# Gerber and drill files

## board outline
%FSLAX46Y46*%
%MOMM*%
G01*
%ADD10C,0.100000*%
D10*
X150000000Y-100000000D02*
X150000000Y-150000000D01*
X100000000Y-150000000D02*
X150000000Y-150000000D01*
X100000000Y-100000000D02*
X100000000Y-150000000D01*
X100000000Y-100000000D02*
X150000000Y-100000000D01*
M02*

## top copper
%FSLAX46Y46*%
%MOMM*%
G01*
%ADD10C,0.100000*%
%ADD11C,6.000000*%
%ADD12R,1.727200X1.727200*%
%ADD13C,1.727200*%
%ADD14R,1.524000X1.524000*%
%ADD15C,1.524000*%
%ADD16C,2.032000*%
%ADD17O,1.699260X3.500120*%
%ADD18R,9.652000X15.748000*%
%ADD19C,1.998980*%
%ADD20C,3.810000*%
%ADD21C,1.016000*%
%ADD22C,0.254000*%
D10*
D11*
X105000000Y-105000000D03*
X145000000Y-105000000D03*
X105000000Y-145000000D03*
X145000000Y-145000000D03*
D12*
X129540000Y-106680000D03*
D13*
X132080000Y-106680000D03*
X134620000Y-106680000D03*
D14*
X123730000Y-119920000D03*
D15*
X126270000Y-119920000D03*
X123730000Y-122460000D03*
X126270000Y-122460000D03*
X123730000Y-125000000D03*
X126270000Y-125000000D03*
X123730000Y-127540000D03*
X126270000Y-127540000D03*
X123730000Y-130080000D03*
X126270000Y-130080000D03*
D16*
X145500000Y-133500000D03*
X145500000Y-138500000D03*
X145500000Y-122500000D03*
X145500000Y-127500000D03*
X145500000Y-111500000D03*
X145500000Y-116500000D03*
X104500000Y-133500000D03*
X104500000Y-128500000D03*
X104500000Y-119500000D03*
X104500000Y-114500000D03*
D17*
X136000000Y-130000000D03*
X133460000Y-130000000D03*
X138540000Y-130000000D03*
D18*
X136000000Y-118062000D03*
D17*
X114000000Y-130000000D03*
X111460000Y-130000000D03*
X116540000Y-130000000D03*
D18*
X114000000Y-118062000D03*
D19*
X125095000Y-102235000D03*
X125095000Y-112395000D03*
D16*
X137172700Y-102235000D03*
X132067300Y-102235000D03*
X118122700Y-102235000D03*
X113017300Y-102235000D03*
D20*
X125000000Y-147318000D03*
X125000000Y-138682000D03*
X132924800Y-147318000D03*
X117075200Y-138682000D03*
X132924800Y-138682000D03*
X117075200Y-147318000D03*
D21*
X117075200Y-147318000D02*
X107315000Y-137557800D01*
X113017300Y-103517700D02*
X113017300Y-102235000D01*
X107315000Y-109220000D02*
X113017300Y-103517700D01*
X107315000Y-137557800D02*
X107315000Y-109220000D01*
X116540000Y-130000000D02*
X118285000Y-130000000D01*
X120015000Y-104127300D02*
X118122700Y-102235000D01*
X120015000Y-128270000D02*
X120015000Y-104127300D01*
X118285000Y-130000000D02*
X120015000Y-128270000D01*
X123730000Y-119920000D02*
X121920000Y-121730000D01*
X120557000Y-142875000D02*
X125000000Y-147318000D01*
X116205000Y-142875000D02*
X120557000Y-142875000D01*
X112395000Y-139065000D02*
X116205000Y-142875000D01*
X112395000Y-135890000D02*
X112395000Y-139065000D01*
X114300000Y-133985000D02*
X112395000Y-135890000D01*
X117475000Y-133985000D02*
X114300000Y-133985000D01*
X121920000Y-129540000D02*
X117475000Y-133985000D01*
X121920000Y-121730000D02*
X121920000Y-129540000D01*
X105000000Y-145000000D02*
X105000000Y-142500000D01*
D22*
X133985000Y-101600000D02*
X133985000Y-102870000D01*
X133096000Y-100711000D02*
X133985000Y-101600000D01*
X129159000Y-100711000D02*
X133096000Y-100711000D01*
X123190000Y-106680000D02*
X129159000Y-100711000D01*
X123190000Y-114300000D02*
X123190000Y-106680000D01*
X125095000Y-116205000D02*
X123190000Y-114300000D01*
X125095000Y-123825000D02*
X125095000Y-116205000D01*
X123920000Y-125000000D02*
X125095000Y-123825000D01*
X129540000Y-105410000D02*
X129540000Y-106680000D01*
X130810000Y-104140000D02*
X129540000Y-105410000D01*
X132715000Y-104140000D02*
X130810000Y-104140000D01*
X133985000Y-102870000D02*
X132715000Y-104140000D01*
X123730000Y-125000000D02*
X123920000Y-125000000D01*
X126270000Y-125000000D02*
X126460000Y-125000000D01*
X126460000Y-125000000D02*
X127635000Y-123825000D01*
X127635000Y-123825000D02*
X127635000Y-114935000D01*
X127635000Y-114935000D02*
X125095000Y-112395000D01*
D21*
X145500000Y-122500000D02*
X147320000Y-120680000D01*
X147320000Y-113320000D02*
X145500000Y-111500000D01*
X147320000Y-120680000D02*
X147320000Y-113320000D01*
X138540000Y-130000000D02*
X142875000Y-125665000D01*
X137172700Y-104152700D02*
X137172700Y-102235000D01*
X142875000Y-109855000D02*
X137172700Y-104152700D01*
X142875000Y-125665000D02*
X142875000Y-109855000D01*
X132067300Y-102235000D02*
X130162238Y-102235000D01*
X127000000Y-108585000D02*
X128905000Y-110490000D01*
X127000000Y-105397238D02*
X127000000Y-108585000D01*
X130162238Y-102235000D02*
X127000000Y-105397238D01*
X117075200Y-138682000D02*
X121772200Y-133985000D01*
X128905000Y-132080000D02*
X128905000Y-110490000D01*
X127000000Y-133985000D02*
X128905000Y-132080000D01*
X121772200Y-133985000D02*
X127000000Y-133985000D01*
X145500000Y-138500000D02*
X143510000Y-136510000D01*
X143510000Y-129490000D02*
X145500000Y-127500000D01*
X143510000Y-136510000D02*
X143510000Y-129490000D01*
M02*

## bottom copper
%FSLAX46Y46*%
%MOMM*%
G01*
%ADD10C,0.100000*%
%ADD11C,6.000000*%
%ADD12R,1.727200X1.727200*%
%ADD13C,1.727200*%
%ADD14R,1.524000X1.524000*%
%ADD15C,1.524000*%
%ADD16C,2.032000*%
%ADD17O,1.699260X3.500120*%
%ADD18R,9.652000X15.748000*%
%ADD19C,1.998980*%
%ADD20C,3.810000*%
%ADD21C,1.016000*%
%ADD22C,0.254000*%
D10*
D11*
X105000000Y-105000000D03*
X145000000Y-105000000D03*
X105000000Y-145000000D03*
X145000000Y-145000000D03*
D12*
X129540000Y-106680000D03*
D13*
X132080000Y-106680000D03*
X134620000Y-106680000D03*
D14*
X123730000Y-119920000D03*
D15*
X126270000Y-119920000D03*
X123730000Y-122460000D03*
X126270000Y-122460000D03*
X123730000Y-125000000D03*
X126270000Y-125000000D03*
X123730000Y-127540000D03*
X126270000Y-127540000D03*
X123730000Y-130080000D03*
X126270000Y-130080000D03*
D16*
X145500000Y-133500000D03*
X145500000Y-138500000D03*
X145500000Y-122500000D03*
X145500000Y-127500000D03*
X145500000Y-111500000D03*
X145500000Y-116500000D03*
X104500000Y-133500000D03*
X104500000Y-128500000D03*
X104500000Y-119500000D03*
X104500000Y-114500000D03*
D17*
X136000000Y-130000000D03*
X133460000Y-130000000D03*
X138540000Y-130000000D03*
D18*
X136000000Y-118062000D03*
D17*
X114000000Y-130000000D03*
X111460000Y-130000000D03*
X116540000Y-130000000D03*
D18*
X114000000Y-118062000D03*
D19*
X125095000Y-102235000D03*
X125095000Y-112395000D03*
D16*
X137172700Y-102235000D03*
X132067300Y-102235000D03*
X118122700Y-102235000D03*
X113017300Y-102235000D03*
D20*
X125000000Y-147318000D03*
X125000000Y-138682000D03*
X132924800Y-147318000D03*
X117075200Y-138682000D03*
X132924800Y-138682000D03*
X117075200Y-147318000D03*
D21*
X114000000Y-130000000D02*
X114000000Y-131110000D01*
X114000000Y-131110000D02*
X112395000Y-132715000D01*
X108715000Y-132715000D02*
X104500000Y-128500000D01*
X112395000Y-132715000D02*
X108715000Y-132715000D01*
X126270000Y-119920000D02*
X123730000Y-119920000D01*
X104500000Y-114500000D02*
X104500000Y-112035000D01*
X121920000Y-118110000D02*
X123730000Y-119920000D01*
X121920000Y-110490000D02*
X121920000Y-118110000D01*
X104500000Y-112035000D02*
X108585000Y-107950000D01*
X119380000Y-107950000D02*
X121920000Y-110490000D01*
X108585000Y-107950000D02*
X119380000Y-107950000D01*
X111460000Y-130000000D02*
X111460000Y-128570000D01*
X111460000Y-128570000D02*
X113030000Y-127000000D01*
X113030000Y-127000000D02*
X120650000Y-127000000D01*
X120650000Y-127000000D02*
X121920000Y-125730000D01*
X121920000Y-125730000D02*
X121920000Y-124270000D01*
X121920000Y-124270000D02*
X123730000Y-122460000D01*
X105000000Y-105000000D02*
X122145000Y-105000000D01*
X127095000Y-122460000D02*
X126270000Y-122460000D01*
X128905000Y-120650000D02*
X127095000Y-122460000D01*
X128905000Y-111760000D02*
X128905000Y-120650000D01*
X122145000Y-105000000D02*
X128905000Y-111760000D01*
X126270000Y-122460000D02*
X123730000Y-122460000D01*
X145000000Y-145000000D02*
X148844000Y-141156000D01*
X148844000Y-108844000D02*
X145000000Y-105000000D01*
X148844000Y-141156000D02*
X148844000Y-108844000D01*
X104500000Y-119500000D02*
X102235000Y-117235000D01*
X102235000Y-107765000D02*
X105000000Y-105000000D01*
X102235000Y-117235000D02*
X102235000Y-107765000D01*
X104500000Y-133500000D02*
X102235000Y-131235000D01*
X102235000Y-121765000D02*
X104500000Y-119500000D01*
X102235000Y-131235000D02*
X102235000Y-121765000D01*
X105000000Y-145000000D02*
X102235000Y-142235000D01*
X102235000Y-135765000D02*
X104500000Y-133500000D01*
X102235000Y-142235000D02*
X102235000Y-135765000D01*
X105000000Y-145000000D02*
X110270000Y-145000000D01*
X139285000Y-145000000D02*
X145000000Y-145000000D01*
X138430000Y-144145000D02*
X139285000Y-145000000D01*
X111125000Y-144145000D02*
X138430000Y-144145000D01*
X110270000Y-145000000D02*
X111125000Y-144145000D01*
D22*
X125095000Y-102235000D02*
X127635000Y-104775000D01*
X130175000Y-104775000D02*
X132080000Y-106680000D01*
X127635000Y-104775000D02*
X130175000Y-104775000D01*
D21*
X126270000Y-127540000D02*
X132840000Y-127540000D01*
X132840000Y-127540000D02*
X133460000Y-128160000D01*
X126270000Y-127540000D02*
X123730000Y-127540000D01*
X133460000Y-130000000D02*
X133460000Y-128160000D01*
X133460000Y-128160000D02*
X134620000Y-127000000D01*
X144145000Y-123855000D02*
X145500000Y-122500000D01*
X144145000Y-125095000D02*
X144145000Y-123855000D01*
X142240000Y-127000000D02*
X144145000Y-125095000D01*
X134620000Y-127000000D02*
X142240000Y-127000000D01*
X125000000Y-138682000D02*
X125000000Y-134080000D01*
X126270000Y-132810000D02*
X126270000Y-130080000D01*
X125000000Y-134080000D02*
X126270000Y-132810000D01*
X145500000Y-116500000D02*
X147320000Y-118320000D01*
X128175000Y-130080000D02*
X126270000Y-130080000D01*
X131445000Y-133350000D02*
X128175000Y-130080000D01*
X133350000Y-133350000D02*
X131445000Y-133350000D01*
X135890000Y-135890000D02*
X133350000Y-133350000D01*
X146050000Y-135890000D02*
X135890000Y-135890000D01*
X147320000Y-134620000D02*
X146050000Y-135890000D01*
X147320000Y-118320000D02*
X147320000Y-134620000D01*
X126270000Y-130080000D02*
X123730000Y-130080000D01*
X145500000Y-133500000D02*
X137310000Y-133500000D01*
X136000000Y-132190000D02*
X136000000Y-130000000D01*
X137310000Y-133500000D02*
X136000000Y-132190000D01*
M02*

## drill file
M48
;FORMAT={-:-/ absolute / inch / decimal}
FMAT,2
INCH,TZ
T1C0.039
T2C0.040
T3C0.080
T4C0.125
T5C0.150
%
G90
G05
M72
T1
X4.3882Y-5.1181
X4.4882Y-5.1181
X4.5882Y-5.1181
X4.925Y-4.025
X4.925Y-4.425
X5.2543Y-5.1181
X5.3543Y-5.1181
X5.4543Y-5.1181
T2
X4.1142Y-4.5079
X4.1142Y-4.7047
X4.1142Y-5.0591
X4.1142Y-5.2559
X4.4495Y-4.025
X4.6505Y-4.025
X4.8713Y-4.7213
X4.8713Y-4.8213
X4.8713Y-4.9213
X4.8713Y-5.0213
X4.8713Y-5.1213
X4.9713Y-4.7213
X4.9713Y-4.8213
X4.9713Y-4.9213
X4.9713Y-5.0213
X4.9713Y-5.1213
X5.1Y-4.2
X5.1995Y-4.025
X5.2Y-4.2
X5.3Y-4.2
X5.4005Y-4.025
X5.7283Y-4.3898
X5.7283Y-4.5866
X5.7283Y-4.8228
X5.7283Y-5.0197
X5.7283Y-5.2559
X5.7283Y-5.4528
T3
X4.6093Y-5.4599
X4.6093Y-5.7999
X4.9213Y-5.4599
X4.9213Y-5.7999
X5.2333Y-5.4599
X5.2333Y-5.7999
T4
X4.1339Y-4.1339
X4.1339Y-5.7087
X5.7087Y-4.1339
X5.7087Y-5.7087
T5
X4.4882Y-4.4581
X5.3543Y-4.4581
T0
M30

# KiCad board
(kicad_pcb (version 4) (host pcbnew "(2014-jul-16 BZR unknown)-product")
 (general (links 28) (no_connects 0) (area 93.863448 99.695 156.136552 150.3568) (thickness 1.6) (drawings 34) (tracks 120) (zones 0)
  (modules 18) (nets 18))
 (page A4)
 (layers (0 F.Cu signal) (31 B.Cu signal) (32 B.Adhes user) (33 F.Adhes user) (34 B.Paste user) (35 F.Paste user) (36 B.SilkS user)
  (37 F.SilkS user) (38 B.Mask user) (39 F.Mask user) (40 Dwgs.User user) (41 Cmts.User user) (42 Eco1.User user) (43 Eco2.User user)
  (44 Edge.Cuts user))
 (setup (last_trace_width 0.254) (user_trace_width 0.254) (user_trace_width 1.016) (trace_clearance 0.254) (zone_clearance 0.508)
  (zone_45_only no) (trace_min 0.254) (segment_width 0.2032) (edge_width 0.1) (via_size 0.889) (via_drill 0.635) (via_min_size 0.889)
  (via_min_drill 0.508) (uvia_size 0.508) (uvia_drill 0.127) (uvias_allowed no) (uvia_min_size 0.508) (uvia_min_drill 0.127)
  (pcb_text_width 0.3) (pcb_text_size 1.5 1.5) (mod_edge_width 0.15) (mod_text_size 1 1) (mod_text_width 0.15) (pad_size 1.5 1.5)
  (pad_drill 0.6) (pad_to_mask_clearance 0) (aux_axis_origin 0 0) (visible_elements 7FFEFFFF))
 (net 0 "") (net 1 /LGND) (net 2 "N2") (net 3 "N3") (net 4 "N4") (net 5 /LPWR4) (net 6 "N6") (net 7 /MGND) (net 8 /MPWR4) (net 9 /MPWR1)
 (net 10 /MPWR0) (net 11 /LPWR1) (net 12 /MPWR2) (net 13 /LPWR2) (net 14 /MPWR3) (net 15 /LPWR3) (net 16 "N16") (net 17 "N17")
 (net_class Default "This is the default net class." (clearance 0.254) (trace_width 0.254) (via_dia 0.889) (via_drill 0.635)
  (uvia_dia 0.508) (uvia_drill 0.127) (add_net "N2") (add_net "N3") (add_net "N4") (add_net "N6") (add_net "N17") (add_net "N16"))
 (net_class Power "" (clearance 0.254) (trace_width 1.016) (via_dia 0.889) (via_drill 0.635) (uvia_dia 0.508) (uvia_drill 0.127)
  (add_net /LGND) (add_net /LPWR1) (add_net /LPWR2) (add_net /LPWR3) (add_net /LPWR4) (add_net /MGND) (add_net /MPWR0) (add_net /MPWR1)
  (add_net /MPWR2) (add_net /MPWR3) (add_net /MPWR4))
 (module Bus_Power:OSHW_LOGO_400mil (layer B.Cu) (at 135.89 120.015)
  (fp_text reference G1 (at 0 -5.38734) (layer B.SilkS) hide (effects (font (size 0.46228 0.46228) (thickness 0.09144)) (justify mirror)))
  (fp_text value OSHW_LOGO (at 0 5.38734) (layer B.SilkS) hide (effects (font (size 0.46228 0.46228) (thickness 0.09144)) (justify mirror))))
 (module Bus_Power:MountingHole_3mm (layer F.Cu) (at 105 105)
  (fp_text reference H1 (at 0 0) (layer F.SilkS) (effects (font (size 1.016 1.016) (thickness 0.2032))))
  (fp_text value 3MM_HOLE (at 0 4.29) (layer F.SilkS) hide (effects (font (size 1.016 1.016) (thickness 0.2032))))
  (pad 1 thru_hole circle (at 0 0) (size 6 6) (drill 3.175) (layers *.Cu *.SilkS) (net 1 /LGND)))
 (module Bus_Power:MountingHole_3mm (layer F.Cu) (at 145 105)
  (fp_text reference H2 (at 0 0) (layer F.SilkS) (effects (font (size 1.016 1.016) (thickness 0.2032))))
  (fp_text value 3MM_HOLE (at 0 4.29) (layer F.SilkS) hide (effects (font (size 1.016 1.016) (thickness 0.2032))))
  (pad 1 thru_hole circle (at 0 0) (size 6 6) (drill 3.175) (layers *.Cu *.SilkS) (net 1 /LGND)))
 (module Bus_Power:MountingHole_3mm (layer F.Cu) (at 105 145)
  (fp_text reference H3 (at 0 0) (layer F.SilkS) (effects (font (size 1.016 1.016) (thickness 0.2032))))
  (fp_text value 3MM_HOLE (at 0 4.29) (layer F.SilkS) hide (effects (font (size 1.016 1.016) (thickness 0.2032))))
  (pad 1 thru_hole circle (at 0 0) (size 6 6) (drill 3.175) (layers *.Cu *.SilkS) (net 1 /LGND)))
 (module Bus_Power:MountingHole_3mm (layer F.Cu) (at 145 145)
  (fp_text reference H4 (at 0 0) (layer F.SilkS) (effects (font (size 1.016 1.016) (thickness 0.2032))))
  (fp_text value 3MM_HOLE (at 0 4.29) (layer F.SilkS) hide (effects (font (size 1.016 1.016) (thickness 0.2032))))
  (pad 1 thru_hole circle (at 0 0) (size 6 6) (drill 3.175) (layers *.Cu *.SilkS) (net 1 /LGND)))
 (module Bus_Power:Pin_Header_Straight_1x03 (layer F.Cu) (at 132.08 106.68)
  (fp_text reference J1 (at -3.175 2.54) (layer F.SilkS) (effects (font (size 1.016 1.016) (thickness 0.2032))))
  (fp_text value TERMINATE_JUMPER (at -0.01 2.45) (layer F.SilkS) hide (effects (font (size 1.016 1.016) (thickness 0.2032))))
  (pad 1 thru_hole rect (at -2.54 0) (size 1.7272 1.7272) (drill 1.016) (layers *.Cu *.Mask F.SilkS) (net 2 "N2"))
  (pad 2 thru_hole circle (at 0 0) (size 1.7272 1.7272) (drill 1.016) (layers *.Cu *.Mask F.SilkS) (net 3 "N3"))
  (pad 3 thru_hole circle (at 2.54 0) (size 1.7272 1.7272) (drill 1.016) (layers *.Cu *.Mask F.SilkS) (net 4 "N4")))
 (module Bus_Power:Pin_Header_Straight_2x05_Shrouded (layer F.Cu) (at 125 125 270)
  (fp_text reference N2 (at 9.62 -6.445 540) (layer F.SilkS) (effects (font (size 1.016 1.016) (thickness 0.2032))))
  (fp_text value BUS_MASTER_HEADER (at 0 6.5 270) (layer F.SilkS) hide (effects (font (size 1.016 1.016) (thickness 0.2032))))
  (pad 1 thru_hole rect (at -5.08 1.27 270) (size 1.524 1.524) (drill 1.016) (layers *.Cu *.Mask F.SilkS) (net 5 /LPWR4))
  (pad 2 thru_hole circle (at -5.08 -1.27 270) (size 1.524 1.524) (drill 1.016) (layers *.Cu *.Mask F.SilkS) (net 5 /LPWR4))
  (pad 3 thru_hole circle (at -2.54 1.27 270) (size 1.524 1.524) (drill 1.016) (layers *.Cu *.Mask F.SilkS) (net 1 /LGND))
  (pad 4 thru_hole circle (at -2.54 -1.27 270) (size 1.524 1.524) (drill 1.016) (layers *.Cu *.Mask F.SilkS) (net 1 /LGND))
  (pad 5 thru_hole circle (at 0 1.27 270) (size 1.524 1.524) (drill 1.016) (layers *.Cu *.Mask F.SilkS) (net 2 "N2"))
  (pad 6 thru_hole circle (at 0 -1.27 270) (size 1.524 1.524) (drill 1.016) (layers *.Cu *.Mask F.SilkS) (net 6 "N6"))
  (pad 7 thru_hole circle (at 2.54 1.27 270) (size 1.524 1.524) (drill 1.016) (layers *.Cu *.Mask F.SilkS) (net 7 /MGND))
  (pad 8 thru_hole circle (at 2.54 -1.27 270) (size 1.524 1.524) (drill 1.016) (layers *.Cu *.Mask F.SilkS) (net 7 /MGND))
  (pad 9 thru_hole circle (at 5.08 1.27 270) (size 1.524 1.524) (drill 1.016) (layers *.Cu *.Mask F.SilkS) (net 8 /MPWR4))
  (pad 10 thru_hole circle (at 5.08 -1.27 270) (size 1.524 1.524) (drill 1.016) (layers *.Cu *.Mask F.SilkS) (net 8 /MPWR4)))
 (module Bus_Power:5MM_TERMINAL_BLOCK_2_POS (layer F.Cu) (at 145.5 136 270)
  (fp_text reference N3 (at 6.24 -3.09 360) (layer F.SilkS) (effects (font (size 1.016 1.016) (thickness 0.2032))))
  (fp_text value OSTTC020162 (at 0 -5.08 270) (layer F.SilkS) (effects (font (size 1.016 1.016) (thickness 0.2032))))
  (pad 1 thru_hole circle (at -2.5 0 270) (size 2.032 2.032) (drill 1.016) (layers *.Cu *.Mask) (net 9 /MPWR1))
  (pad 2 thru_hole circle (at 2.5 0 270) (size 2.032 2.032) (drill 1.016) (layers *.Cu *.Mask) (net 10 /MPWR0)))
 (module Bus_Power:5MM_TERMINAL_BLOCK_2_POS (layer F.Cu) (at 145.5 125 270)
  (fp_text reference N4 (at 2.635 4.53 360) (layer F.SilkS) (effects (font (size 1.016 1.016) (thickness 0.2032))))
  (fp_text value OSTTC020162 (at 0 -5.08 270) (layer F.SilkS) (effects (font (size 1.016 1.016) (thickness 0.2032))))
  (pad 1 thru_hole circle (at -2.5 0 270) (size 2.032 2.032) (drill 1.016) (layers *.Cu *.Mask) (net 7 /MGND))
  (pad 2 thru_hole circle (at 2.5 0 270) (size 2.032 2.032) (drill 1.016) (layers *.Cu *.Mask) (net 10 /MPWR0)))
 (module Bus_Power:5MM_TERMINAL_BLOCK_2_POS (layer F.Cu) (at 145.5 114 270)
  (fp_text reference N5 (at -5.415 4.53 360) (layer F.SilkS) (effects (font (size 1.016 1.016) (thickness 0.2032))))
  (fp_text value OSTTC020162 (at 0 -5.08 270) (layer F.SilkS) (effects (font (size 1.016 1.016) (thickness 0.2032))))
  (pad 1 thru_hole circle (at -2.5 0 270) (size 2.032 2.032) (drill 1.016) (layers *.Cu *.Mask) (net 7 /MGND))
  (pad 2 thru_hole circle (at 2.5 0 270) (size 2.032 2.032) (drill 1.016) (layers *.Cu *.Mask) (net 8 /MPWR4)))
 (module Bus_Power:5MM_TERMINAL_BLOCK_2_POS (layer F.Cu) (at 104.5 131 90)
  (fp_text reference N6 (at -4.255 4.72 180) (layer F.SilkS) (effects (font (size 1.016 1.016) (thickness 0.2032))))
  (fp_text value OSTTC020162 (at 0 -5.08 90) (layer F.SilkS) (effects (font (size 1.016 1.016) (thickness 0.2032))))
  (pad 1 thru_hole circle (at -2.5 0 90) (size 2.032 2.032) (drill 1.016) (layers *.Cu *.Mask) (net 1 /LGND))
  (pad 2 thru_hole circle (at 2.5 0 90) (size 2.032 2.032) (drill 1.016) (layers *.Cu *.Mask) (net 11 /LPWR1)))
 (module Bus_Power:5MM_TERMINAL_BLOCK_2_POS (layer F.Cu) (at 104.5 117 90)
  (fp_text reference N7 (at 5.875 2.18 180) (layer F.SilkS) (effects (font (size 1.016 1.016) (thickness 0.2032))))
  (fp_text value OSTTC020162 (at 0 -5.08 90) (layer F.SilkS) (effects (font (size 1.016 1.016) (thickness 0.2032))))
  (pad 1 thru_hole circle (at -2.5 0 90) (size 2.032 2.032) (drill 1.016) (layers *.Cu *.Mask) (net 1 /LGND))
  (pad 2 thru_hole circle (at 2.5 0 90) (size 2.032 2.032) (drill 1.016) (layers *.Cu *.Mask) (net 5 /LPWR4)))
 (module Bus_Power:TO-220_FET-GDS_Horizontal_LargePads (layer F.Cu) (at 136 130)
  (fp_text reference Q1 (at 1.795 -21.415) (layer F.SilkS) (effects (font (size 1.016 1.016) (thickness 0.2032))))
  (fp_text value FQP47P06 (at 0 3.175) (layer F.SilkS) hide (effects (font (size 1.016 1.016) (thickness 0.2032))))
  (pad D thru_hole oval (at 0 0 90) (size 3.50012 1.69926) (drill 1.00076) (layers *.Cu *.Mask F.SilkS) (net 9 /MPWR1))
  (pad G thru_hole oval (at -2.54 0 90) (size 3.50012 1.69926) (drill 1.00076) (layers *.Cu *.Mask F.SilkS) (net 7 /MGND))
  (pad S thru_hole oval (at 2.54 0 90) (size 3.50012 1.69926) (drill 1.00076) (layers *.Cu *.Mask F.SilkS) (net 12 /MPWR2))
  (pad 2 thru_hole rect (at 0 -16.764 90) (size 15.748 9.652) (drill 3.79984 (offset -4.826 0)) (layers *.Cu F.SilkS F.Mask)))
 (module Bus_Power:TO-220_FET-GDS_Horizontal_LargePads (layer F.Cu) (at 114 130)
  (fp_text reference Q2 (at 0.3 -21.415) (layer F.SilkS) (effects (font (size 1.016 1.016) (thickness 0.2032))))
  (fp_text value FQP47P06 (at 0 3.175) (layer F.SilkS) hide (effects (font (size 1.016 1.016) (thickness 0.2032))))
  (pad D thru_hole oval (at 0 0 90) (size 3.50012 1.69926) (drill 1.00076) (layers *.Cu *.Mask F.SilkS) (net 11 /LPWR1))
  (pad G thru_hole oval (at -2.54 0 90) (size 3.50012 1.69926) (drill 1.00076) (layers *.Cu *.Mask F.SilkS) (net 1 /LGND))
  (pad S thru_hole oval (at 2.54 0 90) (size 3.50012 1.69926) (drill 1.00076) (layers *.Cu *.Mask F.SilkS) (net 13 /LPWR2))
  (pad 2 thru_hole rect (at 0 -16.764 90) (size 15.748 9.652) (drill 3.79984 (offset -4.826 0)) (layers *.Cu F.SilkS F.Mask)))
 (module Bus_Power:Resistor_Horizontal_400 (layer F.Cu) (at 125.095 107.315 270)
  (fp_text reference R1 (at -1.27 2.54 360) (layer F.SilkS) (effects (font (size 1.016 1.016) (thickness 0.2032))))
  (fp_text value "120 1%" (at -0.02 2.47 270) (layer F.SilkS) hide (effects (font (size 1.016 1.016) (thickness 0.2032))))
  (pad 1 thru_hole circle (at -5.08 0 270) (size 1.99898 1.99898) (drill 1.00076) (layers *.Cu *.SilkS *.Mask) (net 3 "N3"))
  (pad 2 thru_hole circle (at 5.08 0 270) (size 1.99898 1.99898) (drill 1.00076) (layers *.Cu *.SilkS *.Mask) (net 6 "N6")))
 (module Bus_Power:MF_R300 (layer F.Cu) (at 134.62 102.235 180)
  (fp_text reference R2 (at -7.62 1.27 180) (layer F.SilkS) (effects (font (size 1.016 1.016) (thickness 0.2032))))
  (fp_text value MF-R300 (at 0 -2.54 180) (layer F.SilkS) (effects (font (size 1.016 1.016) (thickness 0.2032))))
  (pad 1 thru_hole circle (at -2.5527 0 180) (size 2.032 2.032) (drill 1.016) (layers *.Cu *.Mask) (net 12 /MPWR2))
  (pad 2 thru_hole circle (at 2.5527 0 180) (size 2.032 2.032) (drill 1.016) (layers *.Cu *.Mask) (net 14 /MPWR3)))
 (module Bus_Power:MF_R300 (layer F.Cu) (at 115.57 102.235 180)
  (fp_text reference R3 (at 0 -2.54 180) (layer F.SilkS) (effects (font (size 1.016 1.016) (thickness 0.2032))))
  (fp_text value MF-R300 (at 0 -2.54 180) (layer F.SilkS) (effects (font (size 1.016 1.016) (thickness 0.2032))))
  (pad 1 thru_hole circle (at -2.5527 0 180) (size 2.032 2.032) (drill 1.016) (layers *.Cu *.Mask) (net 13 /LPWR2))
  (pad 2 thru_hole circle (at 2.5527 0 180) (size 2.032 2.032) (drill 1.016) (layers *.Cu *.Mask) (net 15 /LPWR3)))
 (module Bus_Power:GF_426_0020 (layer F.Cu) (at 125 143)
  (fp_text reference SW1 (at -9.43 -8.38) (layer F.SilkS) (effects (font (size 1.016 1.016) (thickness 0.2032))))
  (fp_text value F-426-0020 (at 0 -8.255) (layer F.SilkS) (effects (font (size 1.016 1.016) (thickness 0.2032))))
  (pad 5 thru_hole circle (at 0 4.318) (size 3.81 3.81) (drill 2.032) (layers *.Cu *.Mask) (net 5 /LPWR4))
  (pad 2 thru_hole circle (at 0 -4.318) (size 3.81 3.81) (drill 2.032) (layers *.Cu *.Mask) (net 8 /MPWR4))
  (pad 6 thru_hole circle (at 7.9248 4.318) (size 3.81 3.81) (drill 2.032) (layers *.Cu *.Mask) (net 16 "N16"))
  (pad 1 thru_hole circle (at -7.9248 -4.318) (size 3.81 3.81) (drill 2.032) (layers *.Cu *.Mask) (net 14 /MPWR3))
  (pad 3 thru_hole circle (at 7.9248 -4.318) (size 3.81 3.81) (drill 2.032) (layers *.Cu *.Mask) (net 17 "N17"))
  (pad 4 thru_hole circle (at -7.9248 4.318) (size 3.81 3.81) (drill 2.032) (layers *.Cu *.Mask) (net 15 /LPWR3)))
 (gr_line (start 150 100) (end 150 150) (angle 90) (layer Edge.Cuts) (width 0.1))
 (gr_line (start 100 150) (end 150 150) (angle 90) (layer Edge.Cuts) (width 0.1))
 (gr_line (start 100 100) (end 100 150) (angle 90) (layer Edge.Cuts) (width 0.1))
 (gr_line (start 100 100) (end 150 100) (angle 90) (layer Edge.Cuts) (width 0.1))
 (segment (start 114 130) (end 114 131.11) (width 1.016) (layer B.Cu) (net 11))
 (segment (start 114 131.11) (end 112.395 132.715) (width 1.016) (layer B.Cu) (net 11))
 (segment (start 108.715 132.715) (end 104.5 128.5) (width 1.016) (layer B.Cu) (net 11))
 (segment (start 112.395 132.715) (end 108.715 132.715) (width 1.016) (layer B.Cu) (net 11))
 (segment (start 117.0752 147.318) (end 107.315 137.5578) (width 1.016) (layer F.Cu) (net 15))
 (segment (start 113.0173 103.5177) (end 113.0173 102.235) (width 1.016) (layer F.Cu) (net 15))
 (segment (start 107.315 109.22) (end 113.0173 103.5177) (width 1.016) (layer F.Cu) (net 15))
 (segment (start 107.315 137.5578) (end 107.315 109.22) (width 1.016) (layer F.Cu) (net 15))
 (segment (start 116.54 130) (end 118.285 130) (width 1.016) (layer F.Cu) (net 13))
 (segment (start 120.015 104.1273) (end 118.1227 102.235) (width 1.016) (layer F.Cu) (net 13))
 (segment (start 120.015 128.27) (end 120.015 104.1273) (width 1.016) (layer F.Cu) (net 13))
 (segment (start 118.285 130) (end 120.015 128.27) (width 1.016) (layer F.Cu) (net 13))
 (segment (start 126.27 119.92) (end 123.73 119.92) (width 1.016) (layer B.Cu) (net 5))
 (segment (start 123.73 119.92) (end 121.92 121.73) (width 1.016) (layer F.Cu) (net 5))
 (segment (start 120.557 142.875) (end 125 147.318) (width 1.016) (layer F.Cu) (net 5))
 (segment (start 116.205 142.875) (end 120.557 142.875) (width 1.016) (layer F.Cu) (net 5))
 (segment (start 112.395 139.065) (end 116.205 142.875) (width 1.016) (layer F.Cu) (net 5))
 (segment (start 112.395 135.89) (end 112.395 139.065) (width 1.016) (layer F.Cu) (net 5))
 (segment (start 114.3 133.985) (end 112.395 135.89) (width 1.016) (layer F.Cu) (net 5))
 (segment (start 117.475 133.985) (end 114.3 133.985) (width 1.016) (layer F.Cu) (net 5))
 (segment (start 121.92 129.54) (end 117.475 133.985) (width 1.016) (layer F.Cu) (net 5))
 (segment (start 121.92 121.73) (end 121.92 129.54) (width 1.016) (layer F.Cu) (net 5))
 (segment (start 104.5 114.5) (end 104.5 112.035) (width 1.016) (layer B.Cu) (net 5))
 (segment (start 121.92 118.11) (end 123.73 119.92) (width 1.016) (layer B.Cu) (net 5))
 (segment (start 121.92 110.49) (end 121.92 118.11) (width 1.016) (layer B.Cu) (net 5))
 (segment (start 104.5 112.035) (end 108.585 107.95) (width 1.016) (layer B.Cu) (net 5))
 (segment (start 119.38 107.95) (end 121.92 110.49) (width 1.016) (layer B.Cu) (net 5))
 (segment (start 108.585 107.95) (end 119.38 107.95) (width 1.016) (layer B.Cu) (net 5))
 (segment (start 111.46 130) (end 111.46 128.57) (width 1.016) (layer B.Cu) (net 1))
 (segment (start 111.46 128.57) (end 113.03 127) (width 1.016) (layer B.Cu) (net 1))
 (segment (start 113.03 127) (end 120.65 127) (width 1.016) (layer B.Cu) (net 1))
 (segment (start 120.65 127) (end 121.92 125.73) (width 1.016) (layer B.Cu) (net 1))
 (segment (start 121.92 125.73) (end 121.92 124.27) (width 1.016) (layer B.Cu) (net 1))
 (segment (start 121.92 124.27) (end 123.73 122.46) (width 1.016) (layer B.Cu) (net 1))
 (segment (start 105 105) (end 122.145 105) (width 1.016) (layer B.Cu) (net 1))
 (segment (start 127.095 122.46) (end 126.27 122.46) (width 1.016) (layer B.Cu) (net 1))
 (segment (start 128.905 120.65) (end 127.095 122.46) (width 1.016) (layer B.Cu) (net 1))
 (segment (start 128.905 111.76) (end 128.905 120.65) (width 1.016) (layer B.Cu) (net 1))
 (segment (start 122.145 105) (end 128.905 111.76) (width 1.016) (layer B.Cu) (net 1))
 (segment (start 126.27 122.46) (end 123.73 122.46) (width 1.016) (layer B.Cu) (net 1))
 (segment (start 145 145) (end 148.844 141.156) (width 1.016) (layer B.Cu) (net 1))
 (segment (start 148.844 108.844) (end 145 105) (width 1.016) (layer B.Cu) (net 1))
 (segment (start 148.844 141.156) (end 148.844 108.844) (width 1.016) (layer B.Cu) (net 1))
 (segment (start 104.5 119.5) (end 102.235 117.235) (width 1.016) (layer B.Cu) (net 1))
 (segment (start 102.235 107.765) (end 105 105) (width 1.016) (layer B.Cu) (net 1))
 (segment (start 102.235 117.235) (end 102.235 107.765) (width 1.016) (layer B.Cu) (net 1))
 (segment (start 104.5 133.5) (end 102.235 131.235) (width 1.016) (layer B.Cu) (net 1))
 (segment (start 102.235 121.765) (end 104.5 119.5) (width 1.016) (layer B.Cu) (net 1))
 (segment (start 102.235 131.235) (end 102.235 121.765) (width 1.016) (layer B.Cu) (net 1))
 (segment (start 105 145) (end 102.235 142.235) (width 1.016) (layer B.Cu) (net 1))
 (segment (start 102.235 135.765) (end 104.5 133.5) (width 1.016) (layer B.Cu) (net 1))
 (segment (start 102.235 142.235) (end 102.235 135.765) (width 1.016) (layer B.Cu) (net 1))
 (segment (start 105 145) (end 110.27 145) (width 1.016) (layer B.Cu) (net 1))
 (segment (start 139.285 145) (end 145 145) (width 1.016) (layer B.Cu) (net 1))
 (segment (start 138.43 144.145) (end 139.285 145) (width 1.016) (layer B.Cu) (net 1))
 (segment (start 111.125 144.145) (end 138.43 144.145) (width 1.016) (layer B.Cu) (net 1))
 (segment (start 110.27 145) (end 111.125 144.145) (width 1.016) (layer B.Cu) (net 1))
 (segment (start 105 145) (end 105 142.5) (width 1.016) (layer F.Cu) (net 1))
 (segment (start 125.095 102.235) (end 127.635 104.775) (width 0.254) (layer B.Cu) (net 3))
 (segment (start 130.175 104.775) (end 132.08 106.68) (width 0.254) (layer B.Cu) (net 3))
 (segment (start 127.635 104.775) (end 130.175 104.775) (width 0.254) (layer B.Cu) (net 3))
 (segment (start 133.985 101.6) (end 133.985 102.87) (width 0.254) (layer F.Cu) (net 2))
 (segment (start 133.096 100.711) (end 133.985 101.6) (width 0.254) (layer F.Cu) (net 2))
 (segment (start 129.159 100.711) (end 133.096 100.711) (width 0.254) (layer F.Cu) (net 2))
 (segment (start 123.19 106.68) (end 129.159 100.711) (width 0.254) (layer F.Cu) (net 2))
 (segment (start 123.19 114.3) (end 123.19 106.68) (width 0.254) (layer F.Cu) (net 2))
 (segment (start 125.095 116.205) (end 123.19 114.3) (width 0.254) (layer F.Cu) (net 2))
 (segment (start 125.095 123.825) (end 125.095 116.205) (width 0.254) (layer F.Cu) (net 2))
 (segment (start 123.92 125) (end 125.095 123.825) (width 0.254) (layer F.Cu) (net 2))
 (segment (start 129.54 105.41) (end 129.54 106.68) (width 0.254) (layer F.Cu) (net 2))
 (segment (start 130.81 104.14) (end 129.54 105.41) (width 0.254) (layer F.Cu) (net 2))
 (segment (start 132.715 104.14) (end 130.81 104.14) (width 0.254) (layer F.Cu) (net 2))
 (segment (start 133.985 102.87) (end 132.715 104.14) (width 0.254) (layer F.Cu) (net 2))
 (segment (start 123.73 125) (end 123.92 125) (width 0.254) (layer F.Cu) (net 2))
 (segment (start 126.27 125) (end 126.46 125) (width 0.254) (layer F.Cu) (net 6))
 (segment (start 126.46 125) (end 127.635 123.825) (width 0.254) (layer F.Cu) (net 6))
 (segment (start 127.635 123.825) (end 127.635 114.935) (width 0.254) (layer F.Cu) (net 6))
 (segment (start 127.635 114.935) (end 125.095 112.395) (width 0.254) (layer F.Cu) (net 6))
 (segment (start 126.27 127.54) (end 132.84 127.54) (width 1.016) (layer B.Cu) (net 7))
 (segment (start 132.84 127.54) (end 133.46 128.16) (width 1.016) (layer B.Cu) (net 7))
 (segment (start 126.27 127.54) (end 123.73 127.54) (width 1.016) (layer B.Cu) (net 7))
 (segment (start 133.46 130) (end 133.46 128.16) (width 1.016) (layer B.Cu) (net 7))
 (segment (start 133.46 128.16) (end 134.62 127) (width 1.016) (layer B.Cu) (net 7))
 (segment (start 144.145 123.855) (end 145.5 122.5) (width 1.016) (layer B.Cu) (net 7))
 (segment (start 144.145 125.095) (end 144.145 123.855) (width 1.016) (layer B.Cu) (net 7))
 (segment (start 142.24 127) (end 144.145 125.095) (width 1.016) (layer B.Cu) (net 7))
 (segment (start 134.62 127) (end 142.24 127) (width 1.016) (layer B.Cu) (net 7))
 (segment (start 145.5 122.5) (end 147.32 120.68) (width 1.016) (layer F.Cu) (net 7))
 (segment (start 147.32 113.32) (end 145.5 111.5) (width 1.016) (layer F.Cu) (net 7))
 (segment (start 147.32 120.68) (end 147.32 113.32) (width 1.016) (layer F.Cu) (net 7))
 (segment (start 125 138.682) (end 125 134.08) (width 1.016) (layer B.Cu) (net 8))
 (segment (start 126.27 132.81) (end 126.27 130.08) (width 1.016) (layer B.Cu) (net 8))
 (segment (start 125 134.08) (end 126.27 132.81) (width 1.016) (layer B.Cu) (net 8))
 (segment (start 145.5 116.5) (end 147.32 118.32) (width 1.016) (layer B.Cu) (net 8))
 (segment (start 128.175 130.08) (end 126.27 130.08) (width 1.016) (layer B.Cu) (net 8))
 (segment (start 131.445 133.35) (end 128.175 130.08) (width 1.016) (layer B.Cu) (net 8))
 (segment (start 133.35 133.35) (end 131.445 133.35) (width 1.016) (layer B.Cu) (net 8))
 (segment (start 135.89 135.89) (end 133.35 133.35) (width 1.016) (layer B.Cu) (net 8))
 (segment (start 146.05 135.89) (end 135.89 135.89) (width 1.016) (layer B.Cu) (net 8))
 (segment (start 147.32 134.62) (end 146.05 135.89) (width 1.016) (layer B.Cu) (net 8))
 (segment (start 147.32 118.32) (end 147.32 134.62) (width 1.016) (layer B.Cu) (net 8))
 (segment (start 126.27 130.08) (end 123.73 130.08) (width 1.016) (layer B.Cu) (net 8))
 (segment (start 145.5 133.5) (end 137.31 133.5) (width 1.016) (layer B.Cu) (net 9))
 (segment (start 136 132.19) (end 136 130) (width 1.016) (layer B.Cu) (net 9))
 (segment (start 137.31 133.5) (end 136 132.19) (width 1.016) (layer B.Cu) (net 9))
 (segment (start 138.54 130) (end 142.875 125.665) (width 1.016) (layer F.Cu) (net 12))
 (segment (start 137.1727 104.1527) (end 137.1727 102.235) (width 1.016) (layer F.Cu) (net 12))
 (segment (start 142.875 109.855) (end 137.1727 104.1527) (width 1.016) (layer F.Cu) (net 12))
 (segment (start 142.875 125.665) (end 142.875 109.855) (width 1.016) (layer F.Cu) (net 12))
 (segment (start 132.0673 102.235) (end 130.162238 102.235) (width 1.016) (layer F.Cu) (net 14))
 (segment (start 127 108.585) (end 128.905 110.49) (width 1.016) (layer F.Cu) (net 14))
 (segment (start 127 105.397238) (end 127 108.585) (width 1.016) (layer F.Cu) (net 14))
 (segment (start 130.162238 102.235) (end 127 105.397238) (width 1.016) (layer F.Cu) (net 14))
 (segment (start 117.0752 138.682) (end 121.7722 133.985) (width 1.016) (layer F.Cu) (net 14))
 (segment (start 128.905 132.08) (end 128.905 110.49) (width 1.016) (layer F.Cu) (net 14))
 (segment (start 127 133.985) (end 128.905 132.08) (width 1.016) (layer F.Cu) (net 14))
 (segment (start 121.7722 133.985) (end 127 133.985) (width 1.016) (layer F.Cu) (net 14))
 (segment (start 145.5 138.5) (end 143.51 136.51) (width 1.016) (layer F.Cu) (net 10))
 (segment (start 143.51 129.49) (end 145.5 127.5) (width 1.016) (layer F.Cu) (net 10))
 (segment (start 143.51 136.51) (end 143.51 129.49) (width 1.016) (layer F.Cu) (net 10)))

